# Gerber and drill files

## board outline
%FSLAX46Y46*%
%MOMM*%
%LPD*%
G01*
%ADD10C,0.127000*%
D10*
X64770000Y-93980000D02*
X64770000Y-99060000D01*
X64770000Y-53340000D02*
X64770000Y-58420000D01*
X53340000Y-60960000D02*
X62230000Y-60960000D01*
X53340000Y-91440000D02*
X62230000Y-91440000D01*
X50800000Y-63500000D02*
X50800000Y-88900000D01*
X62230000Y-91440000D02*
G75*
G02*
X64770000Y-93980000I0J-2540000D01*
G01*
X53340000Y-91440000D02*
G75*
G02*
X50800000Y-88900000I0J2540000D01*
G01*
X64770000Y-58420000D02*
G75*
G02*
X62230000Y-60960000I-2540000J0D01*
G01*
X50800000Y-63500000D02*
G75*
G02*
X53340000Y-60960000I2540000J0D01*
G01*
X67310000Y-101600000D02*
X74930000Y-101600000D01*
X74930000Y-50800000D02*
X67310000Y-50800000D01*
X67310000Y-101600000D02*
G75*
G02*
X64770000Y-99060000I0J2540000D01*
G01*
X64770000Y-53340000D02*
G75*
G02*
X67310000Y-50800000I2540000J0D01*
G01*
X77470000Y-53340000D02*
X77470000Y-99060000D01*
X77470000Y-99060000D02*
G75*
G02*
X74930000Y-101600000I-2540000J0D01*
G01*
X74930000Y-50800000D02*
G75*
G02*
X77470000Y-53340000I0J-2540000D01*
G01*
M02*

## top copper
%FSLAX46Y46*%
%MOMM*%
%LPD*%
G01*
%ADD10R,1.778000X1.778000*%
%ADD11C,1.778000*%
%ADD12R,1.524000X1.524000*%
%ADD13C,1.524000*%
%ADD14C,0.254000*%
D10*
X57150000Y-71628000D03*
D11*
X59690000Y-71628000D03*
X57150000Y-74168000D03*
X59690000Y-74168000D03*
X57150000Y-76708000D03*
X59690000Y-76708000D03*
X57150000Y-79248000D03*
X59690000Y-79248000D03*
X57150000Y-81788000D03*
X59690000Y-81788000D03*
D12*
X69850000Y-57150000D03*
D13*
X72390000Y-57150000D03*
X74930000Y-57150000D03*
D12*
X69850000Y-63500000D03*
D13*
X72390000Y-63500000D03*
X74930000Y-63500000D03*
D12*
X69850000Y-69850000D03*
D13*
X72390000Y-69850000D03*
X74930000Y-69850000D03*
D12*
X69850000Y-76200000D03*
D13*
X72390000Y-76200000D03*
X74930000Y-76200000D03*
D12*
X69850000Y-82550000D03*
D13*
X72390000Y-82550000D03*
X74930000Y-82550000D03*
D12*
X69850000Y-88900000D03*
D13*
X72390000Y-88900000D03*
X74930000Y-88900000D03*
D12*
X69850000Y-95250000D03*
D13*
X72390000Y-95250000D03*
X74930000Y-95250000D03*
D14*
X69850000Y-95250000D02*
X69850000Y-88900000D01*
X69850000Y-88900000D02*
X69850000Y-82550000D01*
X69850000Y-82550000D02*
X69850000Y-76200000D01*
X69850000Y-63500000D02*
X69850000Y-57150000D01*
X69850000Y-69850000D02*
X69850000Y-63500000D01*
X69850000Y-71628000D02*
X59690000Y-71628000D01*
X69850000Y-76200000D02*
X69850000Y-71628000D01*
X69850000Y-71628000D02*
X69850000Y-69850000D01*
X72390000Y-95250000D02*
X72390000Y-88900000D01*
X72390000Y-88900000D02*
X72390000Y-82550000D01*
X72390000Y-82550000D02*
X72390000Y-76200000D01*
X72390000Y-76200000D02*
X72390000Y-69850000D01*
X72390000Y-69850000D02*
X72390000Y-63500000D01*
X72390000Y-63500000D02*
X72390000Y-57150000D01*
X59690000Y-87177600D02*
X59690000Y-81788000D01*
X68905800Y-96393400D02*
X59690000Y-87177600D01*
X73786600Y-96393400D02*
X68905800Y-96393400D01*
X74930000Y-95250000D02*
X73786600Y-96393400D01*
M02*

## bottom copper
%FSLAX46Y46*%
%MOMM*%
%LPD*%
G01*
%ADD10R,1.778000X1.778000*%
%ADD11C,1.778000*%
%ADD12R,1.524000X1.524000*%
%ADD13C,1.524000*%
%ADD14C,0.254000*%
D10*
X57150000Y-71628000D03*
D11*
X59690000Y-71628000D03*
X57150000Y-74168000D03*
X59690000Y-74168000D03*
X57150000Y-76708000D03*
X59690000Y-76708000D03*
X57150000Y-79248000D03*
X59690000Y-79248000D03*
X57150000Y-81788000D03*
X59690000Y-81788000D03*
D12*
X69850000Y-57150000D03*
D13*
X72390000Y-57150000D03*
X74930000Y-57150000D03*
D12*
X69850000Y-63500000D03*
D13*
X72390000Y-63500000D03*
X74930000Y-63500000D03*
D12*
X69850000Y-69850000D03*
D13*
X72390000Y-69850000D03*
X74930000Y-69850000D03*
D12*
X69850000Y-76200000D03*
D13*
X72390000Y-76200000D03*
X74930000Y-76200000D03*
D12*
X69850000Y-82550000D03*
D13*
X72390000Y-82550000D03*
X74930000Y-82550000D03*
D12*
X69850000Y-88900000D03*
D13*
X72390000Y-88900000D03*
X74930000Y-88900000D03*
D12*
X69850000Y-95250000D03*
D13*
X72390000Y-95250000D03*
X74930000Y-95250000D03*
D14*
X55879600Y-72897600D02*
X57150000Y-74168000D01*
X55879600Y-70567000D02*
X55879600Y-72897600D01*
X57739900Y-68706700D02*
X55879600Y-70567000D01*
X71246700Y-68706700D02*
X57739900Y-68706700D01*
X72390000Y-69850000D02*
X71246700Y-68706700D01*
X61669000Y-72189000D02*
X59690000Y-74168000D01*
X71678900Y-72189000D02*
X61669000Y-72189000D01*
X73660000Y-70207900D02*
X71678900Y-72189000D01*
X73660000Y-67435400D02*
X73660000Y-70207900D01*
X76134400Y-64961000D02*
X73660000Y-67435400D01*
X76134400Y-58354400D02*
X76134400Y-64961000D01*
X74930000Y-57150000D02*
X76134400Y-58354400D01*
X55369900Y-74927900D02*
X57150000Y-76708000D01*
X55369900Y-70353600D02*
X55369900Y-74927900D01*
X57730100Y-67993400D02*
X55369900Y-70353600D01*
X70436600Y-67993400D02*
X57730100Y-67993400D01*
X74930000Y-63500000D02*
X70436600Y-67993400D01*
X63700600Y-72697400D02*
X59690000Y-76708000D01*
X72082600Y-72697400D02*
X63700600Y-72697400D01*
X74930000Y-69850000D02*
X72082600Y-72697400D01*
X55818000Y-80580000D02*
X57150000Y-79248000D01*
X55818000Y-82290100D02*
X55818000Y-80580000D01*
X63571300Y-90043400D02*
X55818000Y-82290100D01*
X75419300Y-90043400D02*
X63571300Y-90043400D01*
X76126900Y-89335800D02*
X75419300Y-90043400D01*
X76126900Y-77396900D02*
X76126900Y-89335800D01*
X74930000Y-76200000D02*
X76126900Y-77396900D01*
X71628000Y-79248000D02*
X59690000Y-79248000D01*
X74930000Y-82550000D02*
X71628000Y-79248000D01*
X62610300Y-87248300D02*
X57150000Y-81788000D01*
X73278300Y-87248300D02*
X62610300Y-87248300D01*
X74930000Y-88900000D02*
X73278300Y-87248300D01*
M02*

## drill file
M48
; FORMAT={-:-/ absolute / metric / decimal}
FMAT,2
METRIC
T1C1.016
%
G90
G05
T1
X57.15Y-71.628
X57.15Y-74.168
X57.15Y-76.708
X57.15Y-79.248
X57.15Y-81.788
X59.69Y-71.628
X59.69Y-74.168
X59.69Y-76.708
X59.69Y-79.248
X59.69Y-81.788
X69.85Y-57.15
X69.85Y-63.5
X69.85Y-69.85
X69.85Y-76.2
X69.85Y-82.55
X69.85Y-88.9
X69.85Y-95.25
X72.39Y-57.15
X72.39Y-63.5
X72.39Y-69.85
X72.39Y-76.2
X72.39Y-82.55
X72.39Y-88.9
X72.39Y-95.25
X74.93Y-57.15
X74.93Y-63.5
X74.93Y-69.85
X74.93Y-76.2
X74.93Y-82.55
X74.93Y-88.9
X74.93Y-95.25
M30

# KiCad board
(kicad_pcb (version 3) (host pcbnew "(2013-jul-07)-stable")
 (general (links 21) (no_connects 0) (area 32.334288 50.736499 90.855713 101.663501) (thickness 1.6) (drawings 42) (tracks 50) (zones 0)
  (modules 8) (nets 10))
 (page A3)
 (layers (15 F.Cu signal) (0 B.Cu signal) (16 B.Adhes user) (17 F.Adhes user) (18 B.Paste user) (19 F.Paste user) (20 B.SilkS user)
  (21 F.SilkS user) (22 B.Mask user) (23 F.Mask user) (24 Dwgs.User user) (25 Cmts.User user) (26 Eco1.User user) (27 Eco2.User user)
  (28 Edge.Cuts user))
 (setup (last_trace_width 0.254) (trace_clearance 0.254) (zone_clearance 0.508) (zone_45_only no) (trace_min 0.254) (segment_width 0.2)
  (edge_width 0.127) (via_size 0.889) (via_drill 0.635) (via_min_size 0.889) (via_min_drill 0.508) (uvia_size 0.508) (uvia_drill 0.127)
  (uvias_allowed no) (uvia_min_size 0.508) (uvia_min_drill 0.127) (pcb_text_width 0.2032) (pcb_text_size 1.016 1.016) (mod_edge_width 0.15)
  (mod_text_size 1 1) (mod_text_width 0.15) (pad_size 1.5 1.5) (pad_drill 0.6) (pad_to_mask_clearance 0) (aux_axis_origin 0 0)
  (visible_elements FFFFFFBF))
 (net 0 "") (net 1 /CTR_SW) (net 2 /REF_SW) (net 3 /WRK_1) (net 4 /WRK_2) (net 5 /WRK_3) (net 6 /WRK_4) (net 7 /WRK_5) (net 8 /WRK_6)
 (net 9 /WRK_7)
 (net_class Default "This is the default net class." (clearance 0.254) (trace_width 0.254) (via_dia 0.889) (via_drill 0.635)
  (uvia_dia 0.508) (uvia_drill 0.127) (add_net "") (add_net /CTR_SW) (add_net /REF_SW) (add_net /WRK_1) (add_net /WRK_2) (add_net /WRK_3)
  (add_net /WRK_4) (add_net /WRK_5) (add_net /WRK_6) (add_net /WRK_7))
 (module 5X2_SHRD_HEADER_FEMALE (layer B.Cu) (at 58.42 76.2 90)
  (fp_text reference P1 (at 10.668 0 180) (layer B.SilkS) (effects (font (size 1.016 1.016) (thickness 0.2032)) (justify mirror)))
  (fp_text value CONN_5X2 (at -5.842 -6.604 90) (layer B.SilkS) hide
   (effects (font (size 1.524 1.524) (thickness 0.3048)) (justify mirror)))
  (pad 1 thru_hole rect (at 4.572 -1.27 270) (size 1.778 1.778) (drill 1.016) (layers *.Cu *.Mask B.SilkS))
  (pad 2 thru_hole circle (at 4.572 1.27 270) (size 1.778 1.778) (drill 1.016) (layers *.Cu *.Mask B.SilkS) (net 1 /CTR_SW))
  (pad 3 thru_hole circle (at 2.032 -1.27 270) (size 1.778 1.778) (drill 1.016) (layers *.Cu *.Mask B.SilkS) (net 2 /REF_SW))
  (pad 4 thru_hole circle (at 2.032 1.27 270) (size 1.778 1.778) (drill 1.016) (layers *.Cu *.Mask B.SilkS) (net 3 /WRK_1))
  (pad 5 thru_hole circle (at -0.508 -1.27 270) (size 1.778 1.778) (drill 1.016) (layers *.Cu *.Mask B.SilkS) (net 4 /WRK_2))
  (pad 6 thru_hole circle (at -0.508 1.27 270) (size 1.778 1.778) (drill 1.016) (layers *.Cu *.Mask B.SilkS) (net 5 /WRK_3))
  (pad 7 thru_hole circle (at -3.048 -1.27 270) (size 1.778 1.778) (drill 1.016) (layers *.Cu *.Mask B.SilkS) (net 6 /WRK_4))
  (pad 8 thru_hole circle (at -3.048 1.27 270) (size 1.778 1.778) (drill 1.016) (layers *.Cu *.Mask B.SilkS) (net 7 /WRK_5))
  (pad 9 thru_hole circle (at -5.588 -1.27 270) (size 1.778 1.778) (drill 1.016) (layers *.Cu *.Mask B.SilkS) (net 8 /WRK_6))
  (pad 10 thru_hole circle (at -5.588 1.27 270) (size 1.778 1.778) (drill 1.016) (layers *.Cu *.Mask B.SilkS) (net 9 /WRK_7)))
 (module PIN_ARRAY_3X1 (layer F.Cu) (at 72.39 57.15)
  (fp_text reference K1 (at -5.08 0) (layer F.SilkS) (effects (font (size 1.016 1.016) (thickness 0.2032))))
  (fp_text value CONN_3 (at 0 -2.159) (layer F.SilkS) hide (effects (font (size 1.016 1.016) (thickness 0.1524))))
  (pad 1 thru_hole rect (at -2.54 0) (size 1.524 1.524) (drill 1.016) (layers *.Cu *.Mask F.SilkS) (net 1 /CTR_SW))
  (pad 2 thru_hole circle (at 0 0) (size 1.524 1.524) (drill 1.016) (layers *.Cu *.Mask F.SilkS) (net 2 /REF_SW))
  (pad 3 thru_hole circle (at 2.54 0) (size 1.524 1.524) (drill 1.016) (layers *.Cu *.Mask F.SilkS) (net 3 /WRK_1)))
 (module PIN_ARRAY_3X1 (layer F.Cu) (at 72.39 63.5)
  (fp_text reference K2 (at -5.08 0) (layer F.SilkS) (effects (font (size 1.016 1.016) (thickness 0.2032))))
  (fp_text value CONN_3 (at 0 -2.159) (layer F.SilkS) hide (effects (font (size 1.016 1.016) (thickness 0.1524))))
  (pad 1 thru_hole rect (at -2.54 0) (size 1.524 1.524) (drill 1.016) (layers *.Cu *.Mask F.SilkS) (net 1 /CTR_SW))
  (pad 2 thru_hole circle (at 0 0) (size 1.524 1.524) (drill 1.016) (layers *.Cu *.Mask F.SilkS) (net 2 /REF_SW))
  (pad 3 thru_hole circle (at 2.54 0) (size 1.524 1.524) (drill 1.016) (layers *.Cu *.Mask F.SilkS) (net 4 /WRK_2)))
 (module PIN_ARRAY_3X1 (layer F.Cu) (at 72.39 69.85)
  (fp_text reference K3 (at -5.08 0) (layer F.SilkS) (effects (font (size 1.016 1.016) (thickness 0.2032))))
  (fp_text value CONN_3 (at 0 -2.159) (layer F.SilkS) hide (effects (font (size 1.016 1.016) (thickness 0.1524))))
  (pad 1 thru_hole rect (at -2.54 0) (size 1.524 1.524) (drill 1.016) (layers *.Cu *.Mask F.SilkS) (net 1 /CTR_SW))
  (pad 2 thru_hole circle (at 0 0) (size 1.524 1.524) (drill 1.016) (layers *.Cu *.Mask F.SilkS) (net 2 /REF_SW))
  (pad 3 thru_hole circle (at 2.54 0) (size 1.524 1.524) (drill 1.016) (layers *.Cu *.Mask F.SilkS) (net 5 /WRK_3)))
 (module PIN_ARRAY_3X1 (layer F.Cu) (at 72.39 76.2)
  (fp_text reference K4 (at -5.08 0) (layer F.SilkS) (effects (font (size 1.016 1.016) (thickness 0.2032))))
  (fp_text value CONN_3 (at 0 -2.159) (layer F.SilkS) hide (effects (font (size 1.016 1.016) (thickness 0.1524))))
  (pad 1 thru_hole rect (at -2.54 0) (size 1.524 1.524) (drill 1.016) (layers *.Cu *.Mask F.SilkS) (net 1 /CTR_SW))
  (pad 2 thru_hole circle (at 0 0) (size 1.524 1.524) (drill 1.016) (layers *.Cu *.Mask F.SilkS) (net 2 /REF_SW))
  (pad 3 thru_hole circle (at 2.54 0) (size 1.524 1.524) (drill 1.016) (layers *.Cu *.Mask F.SilkS) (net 6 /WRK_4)))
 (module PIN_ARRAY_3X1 (layer F.Cu) (at 72.39 82.55)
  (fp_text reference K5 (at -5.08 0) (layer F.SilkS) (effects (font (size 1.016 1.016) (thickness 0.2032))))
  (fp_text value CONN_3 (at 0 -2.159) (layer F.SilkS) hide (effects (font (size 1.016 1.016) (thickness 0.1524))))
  (pad 1 thru_hole rect (at -2.54 0) (size 1.524 1.524) (drill 1.016) (layers *.Cu *.Mask F.SilkS) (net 1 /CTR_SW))
  (pad 2 thru_hole circle (at 0 0) (size 1.524 1.524) (drill 1.016) (layers *.Cu *.Mask F.SilkS) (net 2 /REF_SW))
  (pad 3 thru_hole circle (at 2.54 0) (size 1.524 1.524) (drill 1.016) (layers *.Cu *.Mask F.SilkS) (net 7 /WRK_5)))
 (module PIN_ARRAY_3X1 (layer F.Cu) (at 72.39 88.9)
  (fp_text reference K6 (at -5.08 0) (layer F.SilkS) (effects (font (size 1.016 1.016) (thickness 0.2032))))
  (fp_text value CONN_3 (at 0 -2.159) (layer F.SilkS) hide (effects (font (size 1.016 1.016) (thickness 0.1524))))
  (pad 1 thru_hole rect (at -2.54 0) (size 1.524 1.524) (drill 1.016) (layers *.Cu *.Mask F.SilkS) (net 1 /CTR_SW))
  (pad 2 thru_hole circle (at 0 0) (size 1.524 1.524) (drill 1.016) (layers *.Cu *.Mask F.SilkS) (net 2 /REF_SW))
  (pad 3 thru_hole circle (at 2.54 0) (size 1.524 1.524) (drill 1.016) (layers *.Cu *.Mask F.SilkS) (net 8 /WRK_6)))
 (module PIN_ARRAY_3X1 (layer F.Cu) (at 72.39 95.25)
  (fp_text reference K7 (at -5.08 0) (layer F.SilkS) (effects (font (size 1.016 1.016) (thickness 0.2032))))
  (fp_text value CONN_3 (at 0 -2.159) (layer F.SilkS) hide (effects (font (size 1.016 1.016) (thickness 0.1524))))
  (pad 1 thru_hole rect (at -2.54 0) (size 1.524 1.524) (drill 1.016) (layers *.Cu *.Mask F.SilkS) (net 1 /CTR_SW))
  (pad 2 thru_hole circle (at 0 0) (size 1.524 1.524) (drill 1.016) (layers *.Cu *.Mask F.SilkS) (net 2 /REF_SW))
  (pad 3 thru_hole circle (at 2.54 0) (size 1.524 1.524) (drill 1.016) (layers *.Cu *.Mask F.SilkS) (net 9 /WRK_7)))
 (gr_line (start 64.77 93.98) (end 64.77 99.06) (angle 90) (layer Edge.Cuts) (width 0.127))
 (gr_line (start 64.77 53.34) (end 64.77 58.42) (angle 90) (layer Edge.Cuts) (width 0.127))
 (gr_line (start 53.34 60.96) (end 62.23 60.96) (angle 90) (layer Edge.Cuts) (width 0.127))
 (gr_line (start 53.34 91.44) (end 62.23 91.44) (angle 90) (layer Edge.Cuts) (width 0.127))
 (gr_line (start 50.8 63.5) (end 50.8 88.9) (angle 90) (layer Edge.Cuts) (width 0.127))
 (gr_arc (start 62.23 93.98) (end 62.23 91.44) (angle 90) (layer Edge.Cuts) (width 0.127))
 (gr_arc (start 53.34 88.9) (end 53.34 91.44) (angle 90) (layer Edge.Cuts) (width 0.127))
 (gr_arc (start 62.23 58.42) (end 64.77 58.42) (angle 90) (layer Edge.Cuts) (width 0.127))
 (gr_arc (start 53.34 63.5) (end 50.8 63.5) (angle 90) (layer Edge.Cuts) (width 0.127))
 (gr_line (start 67.31 101.6) (end 74.93 101.6) (angle 90) (layer Edge.Cuts) (width 0.127))
 (gr_line (start 74.93 50.8) (end 67.31 50.8) (angle 90) (layer Edge.Cuts) (width 0.127))
 (gr_arc (start 67.31 99.06) (end 67.31 101.6) (angle 90) (layer Edge.Cuts) (width 0.127))
 (gr_arc (start 67.31 53.34) (end 64.77 53.34) (angle 90) (layer Edge.Cuts) (width 0.127))
 (gr_line (start 77.47 53.34) (end 77.47 99.06) (angle 90) (layer Edge.Cuts) (width 0.127))
 (gr_arc (start 74.93 99.06) (end 77.47 99.06) (angle 90) (layer Edge.Cuts) (width 0.127))
 (gr_arc (start 74.93 53.34) (end 74.93 50.8) (angle 90) (layer Edge.Cuts) (width 0.127))
 (segment (start 69.85 95.25) (end 69.85 88.9) (width 0.254) (layer F.Cu) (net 1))
 (segment (start 69.85 88.9) (end 69.85 82.55) (width 0.254) (layer F.Cu) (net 1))
 (segment (start 69.85 82.55) (end 69.85 76.2) (width 0.254) (layer F.Cu) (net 1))
 (segment (start 69.85 63.5) (end 69.85 57.15) (width 0.254) (layer F.Cu) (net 1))
 (segment (start 69.85 69.85) (end 69.85 63.5) (width 0.254) (layer F.Cu) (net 1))
 (segment (start 69.85 71.628) (end 59.69 71.628) (width 0.254) (layer F.Cu) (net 1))
 (segment (start 69.85 76.2) (end 69.85 71.628) (width 0.254) (layer F.Cu) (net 1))
 (segment (start 69.85 71.628) (end 69.85 69.85) (width 0.254) (layer F.Cu) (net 1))
 (segment (start 72.39 95.25) (end 72.39 88.9) (width 0.254) (layer F.Cu) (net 2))
 (segment (start 72.39 88.9) (end 72.39 82.55) (width 0.254) (layer F.Cu) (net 2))
 (segment (start 72.39 82.55) (end 72.39 76.2) (width 0.254) (layer F.Cu) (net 2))
 (segment (start 72.39 76.2) (end 72.39 69.85) (width 0.254) (layer F.Cu) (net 2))
 (segment (start 72.39 69.85) (end 72.39 63.5) (width 0.254) (layer F.Cu) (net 2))
 (segment (start 72.39 63.5) (end 72.39 57.15) (width 0.254) (layer F.Cu) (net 2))
 (segment (start 55.8796 72.8976) (end 57.15 74.168) (width 0.254) (layer B.Cu) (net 2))
 (segment (start 55.8796 70.567) (end 55.8796 72.8976) (width 0.254) (layer B.Cu) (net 2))
 (segment (start 57.7399 68.7067) (end 55.8796 70.567) (width 0.254) (layer B.Cu) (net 2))
 (segment (start 71.2467 68.7067) (end 57.7399 68.7067) (width 0.254) (layer B.Cu) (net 2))
 (segment (start 72.39 69.85) (end 71.2467 68.7067) (width 0.254) (layer B.Cu) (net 2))
 (segment (start 61.669 72.189) (end 59.69 74.168) (width 0.254) (layer B.Cu) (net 3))
 (segment (start 71.6789 72.189) (end 61.669 72.189) (width 0.254) (layer B.Cu) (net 3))
 (segment (start 73.66 70.2079) (end 71.6789 72.189) (width 0.254) (layer B.Cu) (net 3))
 (segment (start 73.66 67.4354) (end 73.66 70.2079) (width 0.254) (layer B.Cu) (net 3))
 (segment (start 76.1344 64.961) (end 73.66 67.4354) (width 0.254) (layer B.Cu) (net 3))
 (segment (start 76.1344 58.3544) (end 76.1344 64.961) (width 0.254) (layer B.Cu) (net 3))
 (segment (start 74.93 57.15) (end 76.1344 58.3544) (width 0.254) (layer B.Cu) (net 3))
 (segment (start 55.3699 74.9279) (end 57.15 76.708) (width 0.254) (layer B.Cu) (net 4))
 (segment (start 55.3699 70.3536) (end 55.3699 74.9279) (width 0.254) (layer B.Cu) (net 4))
 (segment (start 57.7301 67.9934) (end 55.3699 70.3536) (width 0.254) (layer B.Cu) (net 4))
 (segment (start 70.4366 67.9934) (end 57.7301 67.9934) (width 0.254) (layer B.Cu) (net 4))
 (segment (start 74.93 63.5) (end 70.4366 67.9934) (width 0.254) (layer B.Cu) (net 4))
 (segment (start 63.7006 72.6974) (end 59.69 76.708) (width 0.254) (layer B.Cu) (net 5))
 (segment (start 72.0826 72.6974) (end 63.7006 72.6974) (width 0.254) (layer B.Cu) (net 5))
 (segment (start 74.93 69.85) (end 72.0826 72.6974) (width 0.254) (layer B.Cu) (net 5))
 (segment (start 55.818 80.58) (end 57.15 79.248) (width 0.254) (layer B.Cu) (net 6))
 (segment (start 55.818 82.2901) (end 55.818 80.58) (width 0.254) (layer B.Cu) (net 6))
 (segment (start 63.5713 90.0434) (end 55.818 82.2901) (width 0.254) (layer B.Cu) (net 6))
 (segment (start 75.4193 90.0434) (end 63.5713 90.0434) (width 0.254) (layer B.Cu) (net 6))
 (segment (start 76.1269 89.3358) (end 75.4193 90.0434) (width 0.254) (layer B.Cu) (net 6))
 (segment (start 76.1269 77.3969) (end 76.1269 89.3358) (width 0.254) (layer B.Cu) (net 6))
 (segment (start 74.93 76.2) (end 76.1269 77.3969) (width 0.254) (layer B.Cu) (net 6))
 (segment (start 71.628 79.248) (end 59.69 79.248) (width 0.254) (layer B.Cu) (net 7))
 (segment (start 74.93 82.55) (end 71.628 79.248) (width 0.254) (layer B.Cu) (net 7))
 (segment (start 62.6103 87.2483) (end 57.15 81.788) (width 0.254) (layer B.Cu) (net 8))
 (segment (start 73.2783 87.2483) (end 62.6103 87.2483) (width 0.254) (layer B.Cu) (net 8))
 (segment (start 74.93 88.9) (end 73.2783 87.2483) (width 0.254) (layer B.Cu) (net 8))
 (segment (start 59.69 87.1776) (end 59.69 81.788) (width 0.254) (layer F.Cu) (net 9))
 (segment (start 68.9058 96.3934) (end 59.69 87.1776) (width 0.254) (layer F.Cu) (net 9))
 (segment (start 73.7866 96.3934) (end 68.9058 96.3934) (width 0.254) (layer F.Cu) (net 9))
 (segment (start 74.93 95.25) (end 73.7866 96.3934) (width 0.254) (layer F.Cu) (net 9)))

